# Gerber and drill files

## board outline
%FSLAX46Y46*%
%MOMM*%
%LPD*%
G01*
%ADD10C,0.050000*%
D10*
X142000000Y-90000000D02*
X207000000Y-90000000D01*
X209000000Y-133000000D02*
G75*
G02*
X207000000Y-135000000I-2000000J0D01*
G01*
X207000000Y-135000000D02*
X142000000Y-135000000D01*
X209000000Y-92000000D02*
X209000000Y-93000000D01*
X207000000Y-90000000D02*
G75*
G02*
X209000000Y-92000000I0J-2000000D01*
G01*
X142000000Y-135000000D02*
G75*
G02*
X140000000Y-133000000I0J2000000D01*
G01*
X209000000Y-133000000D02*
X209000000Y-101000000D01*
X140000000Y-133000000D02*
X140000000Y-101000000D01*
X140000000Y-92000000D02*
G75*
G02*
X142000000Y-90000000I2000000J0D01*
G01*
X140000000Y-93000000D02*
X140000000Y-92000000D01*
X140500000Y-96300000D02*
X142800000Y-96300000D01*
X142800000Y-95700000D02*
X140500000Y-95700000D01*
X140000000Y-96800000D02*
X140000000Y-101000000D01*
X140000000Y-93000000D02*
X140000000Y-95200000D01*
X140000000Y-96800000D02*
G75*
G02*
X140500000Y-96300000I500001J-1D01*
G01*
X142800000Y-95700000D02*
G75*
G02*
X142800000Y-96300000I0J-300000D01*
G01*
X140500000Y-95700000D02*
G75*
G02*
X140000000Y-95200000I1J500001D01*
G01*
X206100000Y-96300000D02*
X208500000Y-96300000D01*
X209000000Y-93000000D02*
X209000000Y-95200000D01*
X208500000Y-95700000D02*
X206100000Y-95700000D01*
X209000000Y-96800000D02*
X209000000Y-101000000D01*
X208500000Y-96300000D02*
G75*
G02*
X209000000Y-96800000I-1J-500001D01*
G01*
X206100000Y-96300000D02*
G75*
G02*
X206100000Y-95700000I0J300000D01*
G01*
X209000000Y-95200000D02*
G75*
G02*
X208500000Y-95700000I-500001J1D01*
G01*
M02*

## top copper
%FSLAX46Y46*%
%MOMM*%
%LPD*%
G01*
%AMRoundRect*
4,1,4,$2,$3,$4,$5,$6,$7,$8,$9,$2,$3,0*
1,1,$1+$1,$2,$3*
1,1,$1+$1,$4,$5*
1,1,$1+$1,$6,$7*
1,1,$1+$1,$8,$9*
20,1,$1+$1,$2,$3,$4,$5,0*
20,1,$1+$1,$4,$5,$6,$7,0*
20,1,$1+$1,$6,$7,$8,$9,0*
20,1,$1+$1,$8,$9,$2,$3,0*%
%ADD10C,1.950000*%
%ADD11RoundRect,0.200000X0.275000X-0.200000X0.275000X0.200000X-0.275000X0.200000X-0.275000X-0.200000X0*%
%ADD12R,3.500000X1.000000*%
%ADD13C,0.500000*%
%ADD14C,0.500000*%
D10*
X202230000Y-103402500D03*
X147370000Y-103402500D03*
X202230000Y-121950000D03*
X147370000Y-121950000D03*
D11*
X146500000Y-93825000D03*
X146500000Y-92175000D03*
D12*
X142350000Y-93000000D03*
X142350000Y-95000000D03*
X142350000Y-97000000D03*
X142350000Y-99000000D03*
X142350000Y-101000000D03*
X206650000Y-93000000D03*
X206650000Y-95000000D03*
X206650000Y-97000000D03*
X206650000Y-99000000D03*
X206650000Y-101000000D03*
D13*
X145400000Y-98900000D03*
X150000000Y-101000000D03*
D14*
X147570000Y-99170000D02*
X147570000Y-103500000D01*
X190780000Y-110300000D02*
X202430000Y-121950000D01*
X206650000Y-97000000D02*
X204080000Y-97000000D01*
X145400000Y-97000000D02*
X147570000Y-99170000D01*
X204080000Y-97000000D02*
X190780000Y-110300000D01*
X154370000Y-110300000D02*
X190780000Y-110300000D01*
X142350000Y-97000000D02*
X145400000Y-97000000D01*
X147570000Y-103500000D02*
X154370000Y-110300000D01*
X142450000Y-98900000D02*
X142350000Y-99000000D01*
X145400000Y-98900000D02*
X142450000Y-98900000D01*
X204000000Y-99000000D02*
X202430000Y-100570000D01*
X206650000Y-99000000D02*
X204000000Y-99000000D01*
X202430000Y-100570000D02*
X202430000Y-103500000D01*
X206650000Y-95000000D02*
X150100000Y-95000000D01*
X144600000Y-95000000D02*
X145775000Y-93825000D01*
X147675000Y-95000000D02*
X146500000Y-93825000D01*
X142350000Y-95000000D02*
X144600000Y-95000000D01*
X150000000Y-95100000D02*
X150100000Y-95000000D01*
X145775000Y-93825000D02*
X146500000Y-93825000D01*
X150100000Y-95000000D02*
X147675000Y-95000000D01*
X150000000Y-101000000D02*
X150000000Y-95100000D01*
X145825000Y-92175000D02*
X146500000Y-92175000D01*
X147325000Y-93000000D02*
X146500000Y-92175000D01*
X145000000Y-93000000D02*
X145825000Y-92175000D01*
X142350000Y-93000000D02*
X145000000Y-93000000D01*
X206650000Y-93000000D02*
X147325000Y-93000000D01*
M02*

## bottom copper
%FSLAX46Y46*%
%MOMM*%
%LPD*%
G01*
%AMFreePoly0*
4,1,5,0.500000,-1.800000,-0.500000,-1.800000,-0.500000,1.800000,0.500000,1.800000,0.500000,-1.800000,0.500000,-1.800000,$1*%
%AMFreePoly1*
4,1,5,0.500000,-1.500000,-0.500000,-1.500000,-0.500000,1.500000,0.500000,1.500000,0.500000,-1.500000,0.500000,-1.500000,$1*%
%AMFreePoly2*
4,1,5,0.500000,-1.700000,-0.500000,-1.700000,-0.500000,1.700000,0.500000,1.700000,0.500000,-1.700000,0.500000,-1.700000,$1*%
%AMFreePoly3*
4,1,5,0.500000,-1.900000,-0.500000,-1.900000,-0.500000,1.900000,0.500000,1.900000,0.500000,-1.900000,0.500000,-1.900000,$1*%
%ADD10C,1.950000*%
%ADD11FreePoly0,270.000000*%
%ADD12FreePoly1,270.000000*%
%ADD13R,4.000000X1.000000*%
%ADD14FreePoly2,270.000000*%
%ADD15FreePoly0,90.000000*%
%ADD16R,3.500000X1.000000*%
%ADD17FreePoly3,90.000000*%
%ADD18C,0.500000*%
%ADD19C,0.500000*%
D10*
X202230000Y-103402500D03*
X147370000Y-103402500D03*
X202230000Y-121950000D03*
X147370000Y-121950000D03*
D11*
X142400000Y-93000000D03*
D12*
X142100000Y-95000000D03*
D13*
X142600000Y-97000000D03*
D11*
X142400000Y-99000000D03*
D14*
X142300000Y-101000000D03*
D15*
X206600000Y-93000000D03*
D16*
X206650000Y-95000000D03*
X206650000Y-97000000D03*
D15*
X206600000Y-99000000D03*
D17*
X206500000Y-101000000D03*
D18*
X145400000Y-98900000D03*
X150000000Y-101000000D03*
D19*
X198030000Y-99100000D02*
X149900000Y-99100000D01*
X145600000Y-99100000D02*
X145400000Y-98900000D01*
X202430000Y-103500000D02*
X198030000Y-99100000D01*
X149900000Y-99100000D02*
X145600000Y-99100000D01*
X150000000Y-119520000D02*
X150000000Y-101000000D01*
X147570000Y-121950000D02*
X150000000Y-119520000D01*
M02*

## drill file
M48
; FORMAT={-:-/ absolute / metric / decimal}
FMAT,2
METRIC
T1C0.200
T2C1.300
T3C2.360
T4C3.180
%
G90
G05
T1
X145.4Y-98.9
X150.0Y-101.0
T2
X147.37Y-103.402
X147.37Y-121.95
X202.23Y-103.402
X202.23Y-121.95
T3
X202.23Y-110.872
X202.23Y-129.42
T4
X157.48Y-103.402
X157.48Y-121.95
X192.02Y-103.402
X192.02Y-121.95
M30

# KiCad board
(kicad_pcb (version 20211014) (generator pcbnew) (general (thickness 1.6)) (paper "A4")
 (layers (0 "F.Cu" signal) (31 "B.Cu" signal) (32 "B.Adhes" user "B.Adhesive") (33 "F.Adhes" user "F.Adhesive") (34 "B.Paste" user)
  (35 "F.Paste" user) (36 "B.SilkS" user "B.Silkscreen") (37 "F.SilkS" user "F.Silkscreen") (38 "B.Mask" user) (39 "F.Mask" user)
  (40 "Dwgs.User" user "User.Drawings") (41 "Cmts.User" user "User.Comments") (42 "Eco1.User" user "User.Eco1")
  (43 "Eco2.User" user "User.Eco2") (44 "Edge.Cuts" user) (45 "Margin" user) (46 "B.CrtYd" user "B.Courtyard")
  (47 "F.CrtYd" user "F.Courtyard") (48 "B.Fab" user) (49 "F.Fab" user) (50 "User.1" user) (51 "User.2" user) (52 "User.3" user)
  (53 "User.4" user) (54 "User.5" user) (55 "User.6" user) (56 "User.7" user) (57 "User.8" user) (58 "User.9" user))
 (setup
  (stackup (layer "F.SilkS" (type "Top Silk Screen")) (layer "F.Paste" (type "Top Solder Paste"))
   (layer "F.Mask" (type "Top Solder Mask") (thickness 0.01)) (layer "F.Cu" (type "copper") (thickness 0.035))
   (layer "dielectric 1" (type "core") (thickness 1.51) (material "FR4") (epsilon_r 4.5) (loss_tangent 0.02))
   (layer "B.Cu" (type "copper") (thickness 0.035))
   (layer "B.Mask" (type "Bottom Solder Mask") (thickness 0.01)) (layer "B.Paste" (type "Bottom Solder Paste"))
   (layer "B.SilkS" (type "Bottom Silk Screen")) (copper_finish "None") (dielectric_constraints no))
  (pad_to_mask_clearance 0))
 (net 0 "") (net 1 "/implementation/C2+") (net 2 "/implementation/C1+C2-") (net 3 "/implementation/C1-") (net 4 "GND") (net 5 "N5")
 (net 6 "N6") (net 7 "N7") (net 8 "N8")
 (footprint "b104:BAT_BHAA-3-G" (layer "F.Cu") (at 174.8 103.4025)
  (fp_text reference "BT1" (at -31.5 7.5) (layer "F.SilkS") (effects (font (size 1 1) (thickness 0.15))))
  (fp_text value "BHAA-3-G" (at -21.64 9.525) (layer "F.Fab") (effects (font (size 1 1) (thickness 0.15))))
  (pad "" np_thru_hole circle (at -17.32 0) (size 3.18 3.18) (drill 3.18) (layers *.Cu *.Mask))
  (pad "" np_thru_hole circle (at 27.43 7.47) (size 2.36 2.36) (drill 2.36) (layers *.Cu *.Mask))
  (pad "" np_thru_hole circle (at 17.22 0) (size 3.18 3.18) (drill 3.18) (layers *.Cu *.Mask))
  (pad "+" thru_hole circle (at 27.43 0) (size 1.95 1.95) (drill 1.3) (layers *.Cu *.Mask) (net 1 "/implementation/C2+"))
  (pad "-" thru_hole circle (at -27.43 0) (size 1.95 1.95) (drill 1.3) (layers *.Cu *.Mask) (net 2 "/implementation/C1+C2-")))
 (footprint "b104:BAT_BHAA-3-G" (layer "F.Cu") (at 174.8 121.95)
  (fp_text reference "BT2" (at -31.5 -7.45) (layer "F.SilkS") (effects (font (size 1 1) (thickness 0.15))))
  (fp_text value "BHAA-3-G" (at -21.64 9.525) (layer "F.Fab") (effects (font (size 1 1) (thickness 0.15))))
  (pad "" np_thru_hole circle (at 27.43 7.47) (size 2.36 2.36) (drill 2.36) (layers *.Cu *.Mask))
  (pad "" np_thru_hole circle (at 17.22 0) (size 3.18 3.18) (drill 3.18) (layers *.Cu *.Mask))
  (pad "" np_thru_hole circle (at -17.32 0) (size 3.18 3.18) (drill 3.18) (layers *.Cu *.Mask))
  (pad "+" thru_hole circle (at 27.43 0) (size 1.95 1.95) (drill 1.3) (layers *.Cu *.Mask) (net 2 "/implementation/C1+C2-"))
  (pad "-" thru_hole circle (at -27.43 0) (size 1.95 1.95) (drill 1.3) (layers *.Cu *.Mask) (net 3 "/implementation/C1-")))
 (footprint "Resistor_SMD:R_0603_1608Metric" (layer "F.Cu") (at 146.5 93 90)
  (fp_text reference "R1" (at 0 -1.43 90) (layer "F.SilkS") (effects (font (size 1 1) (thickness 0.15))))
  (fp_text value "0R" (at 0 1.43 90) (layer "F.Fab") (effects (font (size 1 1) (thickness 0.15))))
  (pad "1" smd roundrect (at -0.825 0 90) (size 0.8 0.95) (layers "F.Cu" "F.Paste" "F.Mask") (roundrect_rratio 0.25)
   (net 3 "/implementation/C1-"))
  (pad "2" smd roundrect (at 0.825 0 90) (size 0.8 0.95) (layers "F.Cu" "F.Paste" "F.Mask") (roundrect_rratio 0.25) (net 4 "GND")))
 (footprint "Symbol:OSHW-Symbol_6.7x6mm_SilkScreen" (layer "F.Cu") (at 143.5 131.5)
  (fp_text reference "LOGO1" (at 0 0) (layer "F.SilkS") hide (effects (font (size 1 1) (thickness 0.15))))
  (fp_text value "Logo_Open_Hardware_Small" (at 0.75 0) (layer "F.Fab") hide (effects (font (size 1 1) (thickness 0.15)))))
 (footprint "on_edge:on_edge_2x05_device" (layer "F.Cu") (at 140 97 -90)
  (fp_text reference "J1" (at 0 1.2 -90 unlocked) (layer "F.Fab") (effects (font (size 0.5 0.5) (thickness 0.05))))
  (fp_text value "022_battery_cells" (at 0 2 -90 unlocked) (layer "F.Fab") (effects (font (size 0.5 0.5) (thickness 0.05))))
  (fp_line (start -0.7 -0.5) (end -0.7 -2.8) (layer "Edge.Cuts") (width 0.05))
  (fp_line (start -1.3 -2.8) (end -1.3 -0.5) (layer "Edge.Cuts") (width 0.05))
  (fp_line (start -0.2 0) (end 4 0) (layer "Edge.Cuts") (width 0.05))
  (fp_line (start -4 0) (end -1.8 0) (layer "Edge.Cuts") (width 0.05))
  (fp_arc (start -0.2 0) (mid -0.553553 -0.146447) (end -0.7 -0.5) (layer "Edge.Cuts") (width 0.05))
  (fp_arc (start -1.3 -2.8) (mid -1 -3.1) (end -0.7 -2.8) (layer "Edge.Cuts") (width 0.05))
  (fp_arc (start -1.3 -0.5) (mid -1.446447 -0.146447) (end -1.8 0) (layer "Edge.Cuts") (width 0.05))
  (pad "1" smd rect (at -4 -2.35 90) (size 1 3.5) (layers "F.Cu" "F.Mask") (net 4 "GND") (zone_connect 0))
  (pad "2" smd rect (at -2 -2.35 270) (size 1 3.5) (layers "F.Cu" "F.Mask") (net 3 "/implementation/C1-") (zone_connect 0))
  (pad "3" smd rect (at 0 -2.35 270) (size 1 3.5) (layers "F.Cu" "F.Mask") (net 2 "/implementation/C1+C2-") (zone_connect 0))
  (pad "4" smd rect (at 2 -2.35 90) (size 1 3.5) (layers "F.Cu" "F.Mask") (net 1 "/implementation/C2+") (zone_connect 0))
  (pad "5" smd rect (at 4 -2.35 90) (size 1 3.5) (layers "F.Cu" "F.Mask") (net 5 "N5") (zone_connect 0))
  (pad "6" smd custom (at -4 -2.4 270) (size 1 3.6) (layers "B.Cu" "B.Mask") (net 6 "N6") (zone_connect 0)
   (options (clearance outline) (anchor rect)) (primitives))
  (pad "7" smd custom (at -2 -2.1 270) (size 1 3) (layers "B.Cu" "B.Mask") (zone_connect 0) (options (clearance outline) (anchor rect))
   (primitives))
  (pad "8" smd rect (at 0 -2.6 270) (size 1 4) (layers "B.Cu" "B.Mask") (zone_connect 0))
  (pad "9" smd custom (at 2 -2.4 270) (size 1 3.6) (layers "B.Cu" "B.Mask") (zone_connect 0) (options (clearance outline) (anchor rect))
   (primitives))
  (pad "10" smd custom (at 4 -2.3 270) (size 1 3.4) (layers "B.Cu" "B.Mask") (zone_connect 0) (options (clearance outline) (anchor rect))
   (primitives))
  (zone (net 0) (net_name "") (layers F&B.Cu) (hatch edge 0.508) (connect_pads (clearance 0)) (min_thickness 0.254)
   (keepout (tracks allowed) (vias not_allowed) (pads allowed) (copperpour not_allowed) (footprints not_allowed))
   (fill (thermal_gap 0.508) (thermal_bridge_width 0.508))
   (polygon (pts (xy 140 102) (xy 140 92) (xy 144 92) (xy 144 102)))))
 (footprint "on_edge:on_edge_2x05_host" (layer "F.Cu") (at 209 97 -90)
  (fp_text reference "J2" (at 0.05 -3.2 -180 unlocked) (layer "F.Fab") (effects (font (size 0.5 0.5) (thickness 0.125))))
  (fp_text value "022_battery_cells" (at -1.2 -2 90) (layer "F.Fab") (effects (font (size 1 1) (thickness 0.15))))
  (fp_line (start -0.7 2.9) (end -0.7 0.5) (layer "Edge.Cuts") (width 0.05))
  (fp_line (start -4 0) (end -1.8 0) (layer "Edge.Cuts") (width 0.05))
  (fp_line (start -1.3 0.5) (end -1.3 2.9) (layer "Edge.Cuts") (width 0.05))
  (fp_line (start -0.2 0) (end 4 0) (layer "Edge.Cuts") (width 0.05))
  (fp_arc (start -0.7 0.5) (mid -0.553553 0.146447) (end -0.2 0) (layer "Edge.Cuts") (width 0.05))
  (fp_arc (start -0.7 2.9) (mid -1 3.2) (end -1.3 2.9) (layer "Edge.Cuts") (width 0.05))
  (fp_arc (start -1.8 0) (mid -1.446447 0.146447) (end -1.3 0.5) (layer "Edge.Cuts") (width 0.05))
  (pad "1" smd rect (at -4 2.35 270) (size 1 3.5) (layers "F.Cu" "F.Mask") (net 4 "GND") (zone_connect 0))
  (pad "2" smd rect (at -2 2.35 270) (size 1 3.5) (layers "F.Cu" "F.Mask") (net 3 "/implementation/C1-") (zone_connect 0))
  (pad "3" smd rect (at 0 2.35 270) (size 1 3.5) (layers "F.Cu" "F.Mask") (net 2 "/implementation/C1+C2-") (zone_connect 0))
  (pad "4" smd rect (at 2 2.35 270) (size 1 3.5) (layers "F.Cu" "F.Mask") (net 1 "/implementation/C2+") (zone_connect 0))
  (pad "5" smd rect (at 4 2.35 270) (size 1 3.5) (layers "F.Cu" "F.Mask") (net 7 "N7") (zone_connect 0))
  (pad "6" smd custom (at -4 2.4 90) (size 1 3.6) (layers "B.Cu" "B.Mask") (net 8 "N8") (zone_connect 0)
   (options (clearance outline) (anchor rect)) (primitives))
  (pad "7" smd rect (at -2 2.35 90) (size 1 3.5) (layers "B.Cu" "B.Mask") (zone_connect 0))
  (pad "8" smd rect (at 0 2.35 90) (size 1 3.5) (layers "B.Cu" "B.Mask") (zone_connect 0))
  (pad "9" smd custom (at 2 2.4 90) (size 1 3.6) (layers "B.Cu" "B.Mask") (zone_connect 0) (options (clearance outline) (anchor rect))
   (primitives))
  (pad "10" smd custom (at 4 2.5 90) (size 1 3.8) (layers "B.Cu" "B.Mask") (zone_connect 0) (options (clearance outline) (anchor rect))
   (primitives))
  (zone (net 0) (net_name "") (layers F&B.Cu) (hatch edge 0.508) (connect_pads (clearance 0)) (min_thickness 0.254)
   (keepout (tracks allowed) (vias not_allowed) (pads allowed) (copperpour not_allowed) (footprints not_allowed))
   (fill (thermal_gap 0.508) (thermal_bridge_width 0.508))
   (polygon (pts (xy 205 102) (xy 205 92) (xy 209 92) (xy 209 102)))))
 (gr_line (start 142 90) (end 207 90) (layer "Edge.Cuts") (width 0.05))
 (gr_arc (start 209 133) (mid 208.414214 134.414214) (end 207 135) (layer "Edge.Cuts") (width 0.05))
 (gr_line (start 207 135) (end 142 135) (layer "Edge.Cuts") (width 0.05))
 (gr_line (start 209 92) (end 209 93) (layer "Edge.Cuts") (width 0.05))
 (gr_arc (start 207 90) (mid 208.414214 90.585786) (end 209 92) (layer "Edge.Cuts") (width 0.05))
 (gr_arc (start 142 135) (mid 140.585786 134.414214) (end 140 133) (layer "Edge.Cuts") (width 0.05))
 (gr_line (start 209 133) (end 209 101) (layer "Edge.Cuts") (width 0.05))
 (gr_line (start 140 133) (end 140 101) (layer "Edge.Cuts") (width 0.05))
 (gr_arc (start 140 92) (mid 140.585786 90.585786) (end 142 90) (layer "Edge.Cuts") (width 0.05))
 (gr_line (start 140 93) (end 140 92) (layer "Edge.Cuts") (width 0.05))
 (segment (start 147.57 99.17) (end 147.57 103.5) (width 0.5) (layer "F.Cu") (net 2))
 (segment (start 190.78 110.3) (end 202.43 121.95) (width 0.5) (layer "F.Cu") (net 2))
 (segment (start 206.65 97) (end 204.08 97) (width 0.5) (layer "F.Cu") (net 2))
 (segment (start 145.4 97) (end 147.57 99.17) (width 0.5) (layer "F.Cu") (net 2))
 (segment (start 204.08 97) (end 190.78 110.3) (width 0.5) (layer "F.Cu") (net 2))
 (segment (start 154.37 110.3) (end 190.78 110.3) (width 0.5) (layer "F.Cu") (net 2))
 (segment (start 142.35 97) (end 145.4 97) (width 0.5) (layer "F.Cu") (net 2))
 (segment (start 147.57 103.5) (end 154.37 110.3) (width 0.5) (layer "F.Cu") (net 2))
 (segment (start 142.45 98.9) (end 142.35 99) (width 0.5) (layer "F.Cu") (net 1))
 (segment (start 145.4 98.9) (end 142.45 98.9) (width 0.5) (layer "F.Cu") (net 1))
 (segment (start 204 99) (end 202.43 100.57) (width 0.5) (layer "F.Cu") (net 1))
 (segment (start 206.65 99) (end 204 99) (width 0.5) (layer "F.Cu") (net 1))
 (segment (start 202.43 100.57) (end 202.43 103.5) (width 0.5) (layer "F.Cu") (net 1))
 (via (at 145.4 98.9) (size 0.5) (drill 0.2) (layers "F.Cu" "B.Cu") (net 1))
 (segment (start 198.03 99.1) (end 149.9 99.1) (width 0.5) (layer "B.Cu") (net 1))
 (segment (start 145.6 99.1) (end 145.4 98.9) (width 0.5) (layer "B.Cu") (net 1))
 (segment (start 202.43 103.5) (end 198.03 99.1) (width 0.5) (layer "B.Cu") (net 1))
 (segment (start 149.9 99.1) (end 145.6 99.1) (width 0.5) (layer "B.Cu") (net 1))
 (segment (start 206.65 95) (end 150.1 95) (width 0.5) (layer "F.Cu") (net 3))
 (segment (start 144.6 95) (end 145.775 93.825) (width 0.5) (layer "F.Cu") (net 3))
 (segment (start 147.675 95) (end 146.5 93.825) (width 0.5) (layer "F.Cu") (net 3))
 (segment (start 142.35 95) (end 144.6 95) (width 0.5) (layer "F.Cu") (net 3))
 (segment (start 150 95.1) (end 150.1 95) (width 0.5) (layer "F.Cu") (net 3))
 (segment (start 145.775 93.825) (end 146.5 93.825) (width 0.5) (layer "F.Cu") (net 3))
 (segment (start 150.1 95) (end 147.675 95) (width 0.5) (layer "F.Cu") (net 3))
 (segment (start 150 101) (end 150 95.1) (width 0.5) (layer "F.Cu") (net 3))
 (via (at 150 101) (size 0.5) (drill 0.2) (layers "F.Cu" "B.Cu") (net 3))
 (segment (start 150 119.52) (end 150 101) (width 0.5) (layer "B.Cu") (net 3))
 (segment (start 147.57 121.95) (end 150 119.52) (width 0.5) (layer "B.Cu") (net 3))
 (segment (start 145.825 92.175) (end 146.5 92.175) (width 0.5) (layer "F.Cu") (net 4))
 (segment (start 147.325 93) (end 146.5 92.175) (width 0.5) (layer "F.Cu") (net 4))
 (segment (start 145 93) (end 145.825 92.175) (width 0.5) (layer "F.Cu") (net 4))
 (segment (start 142.35 93) (end 145 93) (width 0.5) (layer "F.Cu") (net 4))
 (segment (start 206.65 93) (end 147.325 93) (width 0.5) (layer "F.Cu") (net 4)))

